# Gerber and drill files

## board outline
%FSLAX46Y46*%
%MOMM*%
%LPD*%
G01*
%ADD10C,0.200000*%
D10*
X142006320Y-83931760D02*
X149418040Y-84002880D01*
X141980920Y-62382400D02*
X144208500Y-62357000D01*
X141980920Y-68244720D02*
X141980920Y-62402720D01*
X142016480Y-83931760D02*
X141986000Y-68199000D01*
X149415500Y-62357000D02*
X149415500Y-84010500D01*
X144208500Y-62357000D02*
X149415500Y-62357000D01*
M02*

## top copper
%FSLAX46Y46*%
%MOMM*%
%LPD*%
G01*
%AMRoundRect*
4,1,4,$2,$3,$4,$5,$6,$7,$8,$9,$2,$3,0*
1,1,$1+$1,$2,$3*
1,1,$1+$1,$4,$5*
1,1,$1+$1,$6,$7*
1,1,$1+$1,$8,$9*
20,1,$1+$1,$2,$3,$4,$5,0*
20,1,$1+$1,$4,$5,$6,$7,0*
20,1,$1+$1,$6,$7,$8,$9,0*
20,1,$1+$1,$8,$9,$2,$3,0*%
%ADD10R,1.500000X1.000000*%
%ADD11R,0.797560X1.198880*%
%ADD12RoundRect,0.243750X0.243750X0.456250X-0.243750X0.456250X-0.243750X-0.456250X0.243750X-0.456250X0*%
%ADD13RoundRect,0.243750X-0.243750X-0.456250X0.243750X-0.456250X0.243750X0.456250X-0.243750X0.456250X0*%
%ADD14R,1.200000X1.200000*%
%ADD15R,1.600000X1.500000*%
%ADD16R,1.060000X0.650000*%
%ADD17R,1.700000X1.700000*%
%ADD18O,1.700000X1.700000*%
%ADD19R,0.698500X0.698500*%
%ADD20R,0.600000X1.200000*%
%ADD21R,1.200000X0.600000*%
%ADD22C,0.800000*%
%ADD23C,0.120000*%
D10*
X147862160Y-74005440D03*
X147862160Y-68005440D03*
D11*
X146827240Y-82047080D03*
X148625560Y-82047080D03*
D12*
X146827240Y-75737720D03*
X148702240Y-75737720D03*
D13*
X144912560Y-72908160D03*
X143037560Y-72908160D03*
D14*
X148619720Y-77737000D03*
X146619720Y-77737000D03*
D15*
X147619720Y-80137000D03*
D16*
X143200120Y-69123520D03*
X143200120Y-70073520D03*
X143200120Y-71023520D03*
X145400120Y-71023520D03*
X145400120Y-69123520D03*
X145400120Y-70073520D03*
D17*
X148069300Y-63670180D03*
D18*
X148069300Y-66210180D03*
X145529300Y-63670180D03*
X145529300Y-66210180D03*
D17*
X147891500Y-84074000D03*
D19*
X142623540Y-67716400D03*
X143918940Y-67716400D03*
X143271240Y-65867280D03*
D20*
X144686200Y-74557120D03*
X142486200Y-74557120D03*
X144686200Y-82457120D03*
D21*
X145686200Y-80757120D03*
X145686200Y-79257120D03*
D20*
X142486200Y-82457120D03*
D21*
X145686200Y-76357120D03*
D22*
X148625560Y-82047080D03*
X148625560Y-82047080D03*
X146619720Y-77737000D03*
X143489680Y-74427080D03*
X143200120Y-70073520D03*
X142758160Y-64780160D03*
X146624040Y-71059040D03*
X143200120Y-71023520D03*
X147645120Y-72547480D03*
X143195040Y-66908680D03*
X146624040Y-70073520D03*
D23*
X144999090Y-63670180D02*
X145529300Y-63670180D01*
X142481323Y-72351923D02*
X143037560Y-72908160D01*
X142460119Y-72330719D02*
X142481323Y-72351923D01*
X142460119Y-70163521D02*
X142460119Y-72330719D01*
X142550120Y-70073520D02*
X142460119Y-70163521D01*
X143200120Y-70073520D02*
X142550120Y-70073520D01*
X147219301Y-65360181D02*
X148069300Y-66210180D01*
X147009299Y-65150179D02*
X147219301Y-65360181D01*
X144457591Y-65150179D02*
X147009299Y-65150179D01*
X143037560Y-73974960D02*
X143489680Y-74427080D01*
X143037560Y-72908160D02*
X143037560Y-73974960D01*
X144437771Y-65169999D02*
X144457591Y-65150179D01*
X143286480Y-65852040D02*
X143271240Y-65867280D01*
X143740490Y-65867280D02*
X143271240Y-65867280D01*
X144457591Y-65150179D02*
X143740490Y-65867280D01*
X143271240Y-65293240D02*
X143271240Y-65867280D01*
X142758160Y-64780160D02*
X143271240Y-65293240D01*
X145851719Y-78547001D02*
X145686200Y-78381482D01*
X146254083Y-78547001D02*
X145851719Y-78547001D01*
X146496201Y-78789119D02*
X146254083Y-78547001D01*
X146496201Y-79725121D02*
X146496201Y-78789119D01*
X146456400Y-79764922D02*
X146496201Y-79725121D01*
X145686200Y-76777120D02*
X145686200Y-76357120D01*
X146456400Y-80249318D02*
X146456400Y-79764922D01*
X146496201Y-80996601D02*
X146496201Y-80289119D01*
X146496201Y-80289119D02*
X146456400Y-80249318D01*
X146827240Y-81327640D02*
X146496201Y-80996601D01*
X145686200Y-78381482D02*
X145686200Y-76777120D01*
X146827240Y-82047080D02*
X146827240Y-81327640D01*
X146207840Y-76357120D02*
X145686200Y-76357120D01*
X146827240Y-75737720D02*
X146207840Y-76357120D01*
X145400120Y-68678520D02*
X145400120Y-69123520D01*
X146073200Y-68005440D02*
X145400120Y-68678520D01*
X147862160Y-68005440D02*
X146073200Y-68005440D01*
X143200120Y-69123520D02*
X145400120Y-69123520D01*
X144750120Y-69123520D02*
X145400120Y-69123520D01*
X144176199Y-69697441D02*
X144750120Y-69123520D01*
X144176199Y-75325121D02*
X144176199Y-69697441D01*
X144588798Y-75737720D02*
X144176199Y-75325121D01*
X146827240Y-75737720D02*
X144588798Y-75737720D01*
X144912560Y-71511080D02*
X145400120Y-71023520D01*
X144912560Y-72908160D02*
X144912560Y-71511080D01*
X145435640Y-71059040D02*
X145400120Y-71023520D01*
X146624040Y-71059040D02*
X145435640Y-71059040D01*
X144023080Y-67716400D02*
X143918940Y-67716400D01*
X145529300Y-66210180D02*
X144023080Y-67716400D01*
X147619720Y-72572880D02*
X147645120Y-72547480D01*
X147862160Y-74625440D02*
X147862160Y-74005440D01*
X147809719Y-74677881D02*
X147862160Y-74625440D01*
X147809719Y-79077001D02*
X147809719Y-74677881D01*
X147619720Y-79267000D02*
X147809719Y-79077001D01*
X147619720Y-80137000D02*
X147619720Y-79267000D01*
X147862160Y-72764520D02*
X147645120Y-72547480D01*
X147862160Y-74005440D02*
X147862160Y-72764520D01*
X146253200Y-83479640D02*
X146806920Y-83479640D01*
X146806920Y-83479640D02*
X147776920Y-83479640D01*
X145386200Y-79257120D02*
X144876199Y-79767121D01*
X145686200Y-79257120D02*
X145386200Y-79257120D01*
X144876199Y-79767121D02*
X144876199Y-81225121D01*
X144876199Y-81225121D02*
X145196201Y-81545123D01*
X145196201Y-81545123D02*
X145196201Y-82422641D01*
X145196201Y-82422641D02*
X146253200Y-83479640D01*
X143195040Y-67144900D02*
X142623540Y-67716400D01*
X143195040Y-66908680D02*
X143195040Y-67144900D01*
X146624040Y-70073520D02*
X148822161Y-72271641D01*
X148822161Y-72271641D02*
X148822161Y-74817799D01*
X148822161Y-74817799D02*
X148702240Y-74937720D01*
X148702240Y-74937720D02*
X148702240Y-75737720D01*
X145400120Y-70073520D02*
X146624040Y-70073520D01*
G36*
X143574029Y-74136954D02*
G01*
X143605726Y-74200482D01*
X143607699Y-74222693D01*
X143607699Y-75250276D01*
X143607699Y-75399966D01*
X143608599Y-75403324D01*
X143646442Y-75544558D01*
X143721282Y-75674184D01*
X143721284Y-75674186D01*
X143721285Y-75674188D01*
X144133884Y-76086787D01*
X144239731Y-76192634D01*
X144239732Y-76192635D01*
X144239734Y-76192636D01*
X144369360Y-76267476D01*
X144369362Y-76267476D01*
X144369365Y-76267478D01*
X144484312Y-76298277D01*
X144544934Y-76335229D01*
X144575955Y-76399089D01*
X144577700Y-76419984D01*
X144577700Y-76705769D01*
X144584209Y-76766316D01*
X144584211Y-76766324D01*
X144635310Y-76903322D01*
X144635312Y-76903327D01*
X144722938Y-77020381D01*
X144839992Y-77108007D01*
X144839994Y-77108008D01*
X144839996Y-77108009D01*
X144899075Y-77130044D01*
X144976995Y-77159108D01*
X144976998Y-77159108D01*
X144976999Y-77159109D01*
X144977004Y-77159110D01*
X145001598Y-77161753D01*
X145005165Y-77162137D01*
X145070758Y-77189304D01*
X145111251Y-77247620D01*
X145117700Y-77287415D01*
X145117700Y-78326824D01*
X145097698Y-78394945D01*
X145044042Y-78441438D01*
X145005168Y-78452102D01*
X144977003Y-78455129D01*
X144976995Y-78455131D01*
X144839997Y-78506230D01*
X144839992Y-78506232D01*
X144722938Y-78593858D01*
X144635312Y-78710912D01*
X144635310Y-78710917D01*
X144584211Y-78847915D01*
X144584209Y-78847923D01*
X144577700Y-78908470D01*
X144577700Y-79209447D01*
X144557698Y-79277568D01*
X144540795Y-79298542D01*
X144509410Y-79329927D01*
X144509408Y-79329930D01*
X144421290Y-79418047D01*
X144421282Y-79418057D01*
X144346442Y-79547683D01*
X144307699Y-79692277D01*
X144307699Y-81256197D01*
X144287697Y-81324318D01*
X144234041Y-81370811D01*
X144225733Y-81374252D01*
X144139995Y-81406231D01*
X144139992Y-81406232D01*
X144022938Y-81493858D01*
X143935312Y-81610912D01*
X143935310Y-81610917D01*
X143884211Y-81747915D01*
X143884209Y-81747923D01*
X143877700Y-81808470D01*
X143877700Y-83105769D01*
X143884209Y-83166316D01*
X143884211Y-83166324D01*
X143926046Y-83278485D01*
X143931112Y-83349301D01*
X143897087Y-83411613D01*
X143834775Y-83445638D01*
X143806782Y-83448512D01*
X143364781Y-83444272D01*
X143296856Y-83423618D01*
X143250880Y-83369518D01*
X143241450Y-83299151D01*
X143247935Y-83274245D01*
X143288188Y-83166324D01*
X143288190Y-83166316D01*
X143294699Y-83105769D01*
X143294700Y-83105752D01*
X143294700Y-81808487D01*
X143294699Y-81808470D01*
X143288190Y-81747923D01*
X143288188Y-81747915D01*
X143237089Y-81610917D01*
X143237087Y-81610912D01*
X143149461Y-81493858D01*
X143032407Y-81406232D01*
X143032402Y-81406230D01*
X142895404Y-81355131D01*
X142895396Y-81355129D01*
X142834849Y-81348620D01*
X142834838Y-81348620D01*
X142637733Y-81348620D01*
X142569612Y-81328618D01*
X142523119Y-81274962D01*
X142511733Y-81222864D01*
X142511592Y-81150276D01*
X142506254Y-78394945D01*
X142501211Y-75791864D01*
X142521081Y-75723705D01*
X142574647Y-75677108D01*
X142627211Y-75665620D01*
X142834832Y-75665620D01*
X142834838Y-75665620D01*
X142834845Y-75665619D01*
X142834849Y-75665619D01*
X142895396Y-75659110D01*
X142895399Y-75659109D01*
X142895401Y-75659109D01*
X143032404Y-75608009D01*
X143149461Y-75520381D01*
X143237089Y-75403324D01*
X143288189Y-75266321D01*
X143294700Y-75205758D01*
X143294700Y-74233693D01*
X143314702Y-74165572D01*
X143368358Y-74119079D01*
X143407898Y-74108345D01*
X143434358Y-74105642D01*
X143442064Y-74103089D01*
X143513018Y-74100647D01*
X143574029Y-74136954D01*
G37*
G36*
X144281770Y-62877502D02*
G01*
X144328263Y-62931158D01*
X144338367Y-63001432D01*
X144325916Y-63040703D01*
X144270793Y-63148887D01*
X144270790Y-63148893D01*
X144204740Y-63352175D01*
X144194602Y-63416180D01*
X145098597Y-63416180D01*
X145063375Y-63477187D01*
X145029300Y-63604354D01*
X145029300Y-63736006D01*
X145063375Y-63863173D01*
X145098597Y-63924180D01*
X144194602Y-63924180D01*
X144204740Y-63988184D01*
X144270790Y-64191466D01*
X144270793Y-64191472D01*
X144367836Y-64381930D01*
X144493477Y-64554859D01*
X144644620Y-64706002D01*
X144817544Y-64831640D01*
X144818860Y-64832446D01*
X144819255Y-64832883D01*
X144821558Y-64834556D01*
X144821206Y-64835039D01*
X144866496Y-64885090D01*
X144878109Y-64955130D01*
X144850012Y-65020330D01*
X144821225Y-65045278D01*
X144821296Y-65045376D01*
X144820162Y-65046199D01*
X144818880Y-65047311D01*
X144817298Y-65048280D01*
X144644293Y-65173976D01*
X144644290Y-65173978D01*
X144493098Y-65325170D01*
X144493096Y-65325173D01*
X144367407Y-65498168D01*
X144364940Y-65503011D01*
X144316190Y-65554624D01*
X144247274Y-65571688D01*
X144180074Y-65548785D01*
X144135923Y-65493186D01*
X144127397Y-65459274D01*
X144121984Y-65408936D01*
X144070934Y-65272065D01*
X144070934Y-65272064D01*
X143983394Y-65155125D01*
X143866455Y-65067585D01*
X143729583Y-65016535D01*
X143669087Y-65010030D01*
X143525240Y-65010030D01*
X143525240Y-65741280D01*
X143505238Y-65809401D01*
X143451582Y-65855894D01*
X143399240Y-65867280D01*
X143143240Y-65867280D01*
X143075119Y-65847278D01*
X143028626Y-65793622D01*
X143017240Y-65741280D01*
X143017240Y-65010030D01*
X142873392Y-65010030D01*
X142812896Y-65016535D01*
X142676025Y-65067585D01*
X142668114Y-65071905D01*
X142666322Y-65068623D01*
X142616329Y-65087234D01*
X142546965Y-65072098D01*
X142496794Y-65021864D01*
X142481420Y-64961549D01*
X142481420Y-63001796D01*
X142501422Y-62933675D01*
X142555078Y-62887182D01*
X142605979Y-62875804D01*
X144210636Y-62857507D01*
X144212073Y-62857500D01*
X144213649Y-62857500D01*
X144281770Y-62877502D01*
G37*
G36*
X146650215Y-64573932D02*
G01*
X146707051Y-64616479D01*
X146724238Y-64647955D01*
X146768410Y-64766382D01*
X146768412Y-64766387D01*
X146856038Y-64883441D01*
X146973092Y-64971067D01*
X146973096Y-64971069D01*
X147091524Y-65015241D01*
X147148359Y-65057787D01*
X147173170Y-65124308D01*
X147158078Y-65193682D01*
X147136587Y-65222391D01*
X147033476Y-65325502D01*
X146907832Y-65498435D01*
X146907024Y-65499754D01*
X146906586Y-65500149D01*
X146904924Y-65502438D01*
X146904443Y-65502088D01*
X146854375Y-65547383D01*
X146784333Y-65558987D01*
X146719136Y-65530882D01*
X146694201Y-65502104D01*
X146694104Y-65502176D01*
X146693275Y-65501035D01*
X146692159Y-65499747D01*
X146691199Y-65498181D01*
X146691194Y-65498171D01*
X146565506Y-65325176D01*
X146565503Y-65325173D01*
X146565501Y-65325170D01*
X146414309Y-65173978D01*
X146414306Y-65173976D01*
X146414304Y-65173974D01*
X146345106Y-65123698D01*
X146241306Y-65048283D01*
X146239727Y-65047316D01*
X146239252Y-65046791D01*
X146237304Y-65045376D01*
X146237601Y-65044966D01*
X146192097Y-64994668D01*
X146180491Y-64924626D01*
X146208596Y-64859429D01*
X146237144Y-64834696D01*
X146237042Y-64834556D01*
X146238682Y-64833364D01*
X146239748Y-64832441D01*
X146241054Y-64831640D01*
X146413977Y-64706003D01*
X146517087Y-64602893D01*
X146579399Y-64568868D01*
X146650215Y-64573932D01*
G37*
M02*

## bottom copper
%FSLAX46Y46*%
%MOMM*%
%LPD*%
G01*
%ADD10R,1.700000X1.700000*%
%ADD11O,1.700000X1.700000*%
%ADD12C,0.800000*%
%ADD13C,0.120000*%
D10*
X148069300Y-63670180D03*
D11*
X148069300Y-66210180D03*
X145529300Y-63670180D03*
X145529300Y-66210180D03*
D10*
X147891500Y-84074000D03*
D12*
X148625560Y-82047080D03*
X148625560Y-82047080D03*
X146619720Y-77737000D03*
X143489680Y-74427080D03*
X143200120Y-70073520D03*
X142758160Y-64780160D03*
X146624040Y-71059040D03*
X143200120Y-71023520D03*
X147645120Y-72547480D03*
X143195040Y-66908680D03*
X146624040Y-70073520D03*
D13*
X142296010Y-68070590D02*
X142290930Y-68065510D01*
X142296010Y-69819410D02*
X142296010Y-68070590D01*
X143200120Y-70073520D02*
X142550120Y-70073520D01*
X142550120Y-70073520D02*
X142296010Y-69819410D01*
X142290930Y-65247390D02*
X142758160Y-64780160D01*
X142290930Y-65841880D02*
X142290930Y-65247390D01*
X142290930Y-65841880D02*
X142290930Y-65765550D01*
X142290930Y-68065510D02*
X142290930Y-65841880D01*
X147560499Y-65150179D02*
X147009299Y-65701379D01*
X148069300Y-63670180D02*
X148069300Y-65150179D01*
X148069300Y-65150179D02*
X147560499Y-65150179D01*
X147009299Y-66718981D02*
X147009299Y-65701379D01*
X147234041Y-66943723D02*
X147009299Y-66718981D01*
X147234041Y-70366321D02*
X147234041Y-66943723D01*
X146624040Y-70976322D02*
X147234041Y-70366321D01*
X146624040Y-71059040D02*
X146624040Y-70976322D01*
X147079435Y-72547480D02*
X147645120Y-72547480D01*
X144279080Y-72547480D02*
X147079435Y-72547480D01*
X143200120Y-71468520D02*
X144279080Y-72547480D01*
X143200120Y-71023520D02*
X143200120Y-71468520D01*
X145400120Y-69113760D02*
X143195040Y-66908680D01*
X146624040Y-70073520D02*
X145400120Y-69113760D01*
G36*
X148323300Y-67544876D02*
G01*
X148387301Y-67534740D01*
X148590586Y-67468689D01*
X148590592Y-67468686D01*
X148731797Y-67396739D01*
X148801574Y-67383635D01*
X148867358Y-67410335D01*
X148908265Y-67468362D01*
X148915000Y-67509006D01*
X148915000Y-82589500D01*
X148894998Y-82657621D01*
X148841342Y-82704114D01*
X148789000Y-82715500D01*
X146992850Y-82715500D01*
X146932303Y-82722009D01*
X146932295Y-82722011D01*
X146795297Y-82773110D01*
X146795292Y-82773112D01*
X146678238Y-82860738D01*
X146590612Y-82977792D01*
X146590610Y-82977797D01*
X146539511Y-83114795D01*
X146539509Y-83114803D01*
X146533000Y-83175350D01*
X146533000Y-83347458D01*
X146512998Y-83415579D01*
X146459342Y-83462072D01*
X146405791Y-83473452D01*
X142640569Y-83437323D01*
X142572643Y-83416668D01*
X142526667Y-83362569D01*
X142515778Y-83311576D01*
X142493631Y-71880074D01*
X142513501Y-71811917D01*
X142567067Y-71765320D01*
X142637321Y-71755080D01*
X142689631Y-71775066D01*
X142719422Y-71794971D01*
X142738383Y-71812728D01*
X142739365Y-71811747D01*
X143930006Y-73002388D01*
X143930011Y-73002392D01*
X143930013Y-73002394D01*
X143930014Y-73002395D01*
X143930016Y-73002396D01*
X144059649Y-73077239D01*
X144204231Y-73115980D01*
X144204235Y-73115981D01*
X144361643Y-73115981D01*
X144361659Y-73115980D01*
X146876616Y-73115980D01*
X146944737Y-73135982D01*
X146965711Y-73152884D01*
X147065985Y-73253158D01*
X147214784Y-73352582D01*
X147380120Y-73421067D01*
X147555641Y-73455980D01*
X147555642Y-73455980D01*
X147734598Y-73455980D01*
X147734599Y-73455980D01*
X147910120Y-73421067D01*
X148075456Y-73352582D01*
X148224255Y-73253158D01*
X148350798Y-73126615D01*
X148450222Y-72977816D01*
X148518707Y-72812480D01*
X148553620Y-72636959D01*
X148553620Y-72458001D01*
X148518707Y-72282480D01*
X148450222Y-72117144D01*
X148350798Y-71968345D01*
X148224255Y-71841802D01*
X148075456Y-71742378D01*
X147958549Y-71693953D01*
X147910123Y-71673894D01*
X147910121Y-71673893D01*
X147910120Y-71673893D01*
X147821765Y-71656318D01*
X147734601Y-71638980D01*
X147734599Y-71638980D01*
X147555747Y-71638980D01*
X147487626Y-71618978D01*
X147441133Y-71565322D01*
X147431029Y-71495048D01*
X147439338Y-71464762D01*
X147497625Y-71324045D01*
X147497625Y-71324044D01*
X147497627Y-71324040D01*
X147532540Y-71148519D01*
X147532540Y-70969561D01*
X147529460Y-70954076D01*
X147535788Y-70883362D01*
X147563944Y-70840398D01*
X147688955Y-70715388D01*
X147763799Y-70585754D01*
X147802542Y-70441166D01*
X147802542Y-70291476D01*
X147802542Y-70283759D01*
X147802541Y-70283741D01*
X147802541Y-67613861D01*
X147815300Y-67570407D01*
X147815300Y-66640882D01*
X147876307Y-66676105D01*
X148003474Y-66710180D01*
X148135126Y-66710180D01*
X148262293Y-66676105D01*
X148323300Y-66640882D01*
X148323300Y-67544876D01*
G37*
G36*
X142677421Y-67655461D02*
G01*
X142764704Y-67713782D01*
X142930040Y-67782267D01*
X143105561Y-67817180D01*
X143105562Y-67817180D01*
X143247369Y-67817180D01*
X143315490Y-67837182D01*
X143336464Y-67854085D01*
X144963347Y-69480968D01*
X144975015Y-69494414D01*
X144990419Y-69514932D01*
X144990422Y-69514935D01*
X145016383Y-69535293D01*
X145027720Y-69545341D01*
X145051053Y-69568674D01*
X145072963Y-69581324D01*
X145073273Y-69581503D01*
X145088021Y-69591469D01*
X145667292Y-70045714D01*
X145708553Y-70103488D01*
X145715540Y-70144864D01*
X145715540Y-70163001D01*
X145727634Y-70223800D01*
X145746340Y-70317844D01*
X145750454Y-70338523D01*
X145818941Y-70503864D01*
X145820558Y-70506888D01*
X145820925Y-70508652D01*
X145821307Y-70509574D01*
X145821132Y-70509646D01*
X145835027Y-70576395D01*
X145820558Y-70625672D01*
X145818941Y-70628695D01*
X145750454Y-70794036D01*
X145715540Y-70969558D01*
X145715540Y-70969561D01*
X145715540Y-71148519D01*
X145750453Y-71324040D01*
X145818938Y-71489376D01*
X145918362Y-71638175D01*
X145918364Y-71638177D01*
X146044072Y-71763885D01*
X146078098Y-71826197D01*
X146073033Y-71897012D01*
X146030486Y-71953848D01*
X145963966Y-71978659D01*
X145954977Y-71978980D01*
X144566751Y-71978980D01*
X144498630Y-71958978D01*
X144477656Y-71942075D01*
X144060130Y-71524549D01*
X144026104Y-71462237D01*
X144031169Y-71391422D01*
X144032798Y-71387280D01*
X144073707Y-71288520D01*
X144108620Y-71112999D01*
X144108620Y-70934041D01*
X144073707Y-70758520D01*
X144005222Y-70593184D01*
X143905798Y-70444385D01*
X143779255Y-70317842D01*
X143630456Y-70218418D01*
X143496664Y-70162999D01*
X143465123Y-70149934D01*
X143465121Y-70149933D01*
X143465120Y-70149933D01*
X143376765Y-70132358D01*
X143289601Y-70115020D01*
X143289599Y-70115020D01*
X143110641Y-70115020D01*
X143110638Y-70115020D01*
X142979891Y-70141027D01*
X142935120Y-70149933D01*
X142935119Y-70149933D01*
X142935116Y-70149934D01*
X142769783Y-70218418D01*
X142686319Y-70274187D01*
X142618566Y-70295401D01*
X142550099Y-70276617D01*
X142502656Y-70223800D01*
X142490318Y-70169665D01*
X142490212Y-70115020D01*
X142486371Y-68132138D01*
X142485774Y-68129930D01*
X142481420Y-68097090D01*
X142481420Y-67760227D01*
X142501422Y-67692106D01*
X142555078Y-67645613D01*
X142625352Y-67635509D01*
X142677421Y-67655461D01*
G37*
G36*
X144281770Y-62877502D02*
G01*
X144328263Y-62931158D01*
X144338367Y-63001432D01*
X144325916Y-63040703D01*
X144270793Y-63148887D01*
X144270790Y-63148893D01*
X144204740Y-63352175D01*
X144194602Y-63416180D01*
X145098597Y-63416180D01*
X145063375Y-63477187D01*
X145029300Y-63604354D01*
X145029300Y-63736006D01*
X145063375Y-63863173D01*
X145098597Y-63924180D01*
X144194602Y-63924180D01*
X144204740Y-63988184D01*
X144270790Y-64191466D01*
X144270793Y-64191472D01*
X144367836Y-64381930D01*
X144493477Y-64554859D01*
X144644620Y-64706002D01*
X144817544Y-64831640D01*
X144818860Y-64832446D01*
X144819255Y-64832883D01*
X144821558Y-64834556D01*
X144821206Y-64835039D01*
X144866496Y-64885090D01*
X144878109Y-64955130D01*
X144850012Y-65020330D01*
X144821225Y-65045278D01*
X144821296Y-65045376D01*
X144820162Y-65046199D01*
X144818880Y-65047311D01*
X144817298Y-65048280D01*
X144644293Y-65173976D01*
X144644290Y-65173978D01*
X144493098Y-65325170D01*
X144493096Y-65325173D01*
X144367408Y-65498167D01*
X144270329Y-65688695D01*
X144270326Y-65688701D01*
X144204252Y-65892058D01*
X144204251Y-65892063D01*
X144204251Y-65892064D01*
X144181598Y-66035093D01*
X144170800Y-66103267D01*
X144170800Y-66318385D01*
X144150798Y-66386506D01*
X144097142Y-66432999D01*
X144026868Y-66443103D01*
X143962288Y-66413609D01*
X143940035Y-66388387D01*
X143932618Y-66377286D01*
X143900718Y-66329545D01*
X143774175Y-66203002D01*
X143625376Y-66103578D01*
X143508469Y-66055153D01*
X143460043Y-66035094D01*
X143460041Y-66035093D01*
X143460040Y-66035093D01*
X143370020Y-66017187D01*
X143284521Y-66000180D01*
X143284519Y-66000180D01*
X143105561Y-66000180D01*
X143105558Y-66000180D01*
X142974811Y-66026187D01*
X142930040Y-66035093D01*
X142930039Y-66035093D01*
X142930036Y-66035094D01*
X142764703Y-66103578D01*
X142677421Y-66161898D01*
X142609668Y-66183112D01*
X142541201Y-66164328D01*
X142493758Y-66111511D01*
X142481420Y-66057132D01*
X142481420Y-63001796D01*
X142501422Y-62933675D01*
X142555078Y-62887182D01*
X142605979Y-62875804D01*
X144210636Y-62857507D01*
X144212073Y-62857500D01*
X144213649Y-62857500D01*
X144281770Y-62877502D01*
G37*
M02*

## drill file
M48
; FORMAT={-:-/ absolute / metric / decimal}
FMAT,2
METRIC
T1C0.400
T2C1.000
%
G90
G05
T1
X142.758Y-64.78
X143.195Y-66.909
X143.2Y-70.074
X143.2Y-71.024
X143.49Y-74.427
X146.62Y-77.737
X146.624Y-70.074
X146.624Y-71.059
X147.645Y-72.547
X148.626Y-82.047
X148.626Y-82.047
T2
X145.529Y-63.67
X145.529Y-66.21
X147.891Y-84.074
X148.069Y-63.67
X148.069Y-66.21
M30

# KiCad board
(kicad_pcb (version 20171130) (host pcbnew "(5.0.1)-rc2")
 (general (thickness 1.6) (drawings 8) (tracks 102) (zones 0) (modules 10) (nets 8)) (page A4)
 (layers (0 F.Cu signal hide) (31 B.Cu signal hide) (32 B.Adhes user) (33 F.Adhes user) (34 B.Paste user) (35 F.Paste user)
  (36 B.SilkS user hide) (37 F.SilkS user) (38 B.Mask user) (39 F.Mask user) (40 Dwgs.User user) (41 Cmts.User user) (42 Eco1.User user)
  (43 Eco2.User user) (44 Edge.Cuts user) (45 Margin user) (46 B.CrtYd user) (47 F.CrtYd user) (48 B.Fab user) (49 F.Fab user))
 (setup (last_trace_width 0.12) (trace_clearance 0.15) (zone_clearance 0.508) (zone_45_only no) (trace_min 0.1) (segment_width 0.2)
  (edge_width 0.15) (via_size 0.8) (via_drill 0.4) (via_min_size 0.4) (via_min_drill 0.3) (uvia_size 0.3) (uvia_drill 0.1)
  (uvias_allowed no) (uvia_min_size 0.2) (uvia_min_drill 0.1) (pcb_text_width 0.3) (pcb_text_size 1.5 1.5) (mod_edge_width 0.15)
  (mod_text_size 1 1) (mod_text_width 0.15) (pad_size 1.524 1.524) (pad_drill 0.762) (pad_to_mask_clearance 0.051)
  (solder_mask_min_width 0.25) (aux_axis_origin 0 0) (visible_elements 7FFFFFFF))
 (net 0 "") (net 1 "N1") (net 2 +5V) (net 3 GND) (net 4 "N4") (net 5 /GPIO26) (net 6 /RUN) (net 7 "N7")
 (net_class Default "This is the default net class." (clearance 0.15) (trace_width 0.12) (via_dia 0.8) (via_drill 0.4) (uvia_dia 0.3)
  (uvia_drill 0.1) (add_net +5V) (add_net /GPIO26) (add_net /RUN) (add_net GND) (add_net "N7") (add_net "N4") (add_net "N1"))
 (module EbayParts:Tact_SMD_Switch (layer F.Cu) (at 149.36216 74.00544 90)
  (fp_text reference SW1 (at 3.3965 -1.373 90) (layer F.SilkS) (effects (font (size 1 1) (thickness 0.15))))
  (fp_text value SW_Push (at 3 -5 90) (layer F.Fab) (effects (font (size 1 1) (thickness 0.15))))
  (pad 1 smd rect (at 0 -1.5 90) (size 1 1.5) (layers F.Cu F.Paste F.Mask) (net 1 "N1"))
  (pad 2 smd rect (at 6 -1.5 90) (size 1 1.5) (layers F.Cu F.Paste F.Mask) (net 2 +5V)))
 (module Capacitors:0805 (layer F.Cu) (at 147.7264 82.04708 180)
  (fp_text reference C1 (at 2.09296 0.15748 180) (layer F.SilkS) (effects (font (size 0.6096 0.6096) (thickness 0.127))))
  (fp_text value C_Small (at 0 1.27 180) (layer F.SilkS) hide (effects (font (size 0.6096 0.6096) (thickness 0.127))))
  (pad 2 smd rect (at 0.89916 0 180) (size 0.79756 1.19888) (layers F.Cu F.Paste F.Mask) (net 2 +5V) (solder_mask_margin 0.1016))
  (pad 1 smd rect (at -0.89916 0 180) (size 0.79756 1.19888) (layers F.Cu F.Paste F.Mask) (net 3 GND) (solder_mask_margin 0.1016)))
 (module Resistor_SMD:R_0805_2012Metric (layer F.Cu) (at 147.76474 75.73772 180)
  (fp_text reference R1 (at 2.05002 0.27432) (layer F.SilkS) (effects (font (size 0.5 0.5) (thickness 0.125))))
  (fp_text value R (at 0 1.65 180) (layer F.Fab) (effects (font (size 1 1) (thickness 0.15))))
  (pad 2 smd roundrect (at 0.9375 0 180) (size 0.975 1.4) (layers F.Cu F.Paste F.Mask) (roundrect_rratio 0.25) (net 2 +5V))
  (pad 1 smd roundrect (at -0.9375 0 180) (size 0.975 1.4) (layers F.Cu F.Paste F.Mask) (roundrect_rratio 0.25) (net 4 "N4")))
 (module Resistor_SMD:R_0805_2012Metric (layer F.Cu) (at 143.97506 72.90816)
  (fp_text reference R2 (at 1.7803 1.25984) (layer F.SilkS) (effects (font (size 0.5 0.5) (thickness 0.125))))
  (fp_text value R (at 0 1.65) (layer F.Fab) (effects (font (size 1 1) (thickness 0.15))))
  (pad 2 smd roundrect (at 0.9375 0) (size 0.975 1.4) (layers F.Cu F.Paste F.Mask) (roundrect_rratio 0.25) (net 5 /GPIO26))
  (pad 1 smd roundrect (at -0.9375 0) (size 0.975 1.4) (layers F.Cu F.Paste F.Mask) (roundrect_rratio 0.25) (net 3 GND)))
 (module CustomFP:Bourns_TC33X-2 (layer F.Cu) (at 147.61972 80.137 180)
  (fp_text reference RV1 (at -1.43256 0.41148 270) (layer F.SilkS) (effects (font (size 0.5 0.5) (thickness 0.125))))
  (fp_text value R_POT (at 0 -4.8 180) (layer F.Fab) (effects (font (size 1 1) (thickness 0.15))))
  (pad 3 smd rect (at -1 2.4 180) (size 1.2 1.2) (layers F.Cu F.Paste F.Mask))
  (pad 2 smd rect (at 1 2.4 180) (size 1.2 1.2) (layers F.Cu F.Paste F.Mask) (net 3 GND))
  (pad 1 smd rect (at 0 0 180) (size 1.6 1.5) (layers F.Cu F.Paste F.Mask) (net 1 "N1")))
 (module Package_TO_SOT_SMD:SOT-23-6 (layer F.Cu) (at 144.30012 70.07352)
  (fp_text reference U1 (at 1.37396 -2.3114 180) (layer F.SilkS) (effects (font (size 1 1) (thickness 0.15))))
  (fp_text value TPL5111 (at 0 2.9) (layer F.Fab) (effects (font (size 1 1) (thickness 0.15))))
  (pad 1 smd rect (at -1.1 -0.95) (size 1.06 0.65) (layers F.Cu F.Paste F.Mask) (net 2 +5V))
  (pad 2 smd rect (at -1.1 0) (size 1.06 0.65) (layers F.Cu F.Paste F.Mask) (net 3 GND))
  (pad 3 smd rect (at -1.1 0.95) (size 1.06 0.65) (layers F.Cu F.Paste F.Mask) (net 1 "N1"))
  (pad 4 smd rect (at 1.1 0.95) (size 1.06 0.65) (layers F.Cu F.Paste F.Mask) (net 5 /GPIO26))
  (pad 6 smd rect (at 1.1 -0.95) (size 1.06 0.65) (layers F.Cu F.Paste F.Mask) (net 2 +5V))
  (pad 5 smd rect (at 1.1 0) (size 1.06 0.65) (layers F.Cu F.Paste F.Mask) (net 4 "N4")))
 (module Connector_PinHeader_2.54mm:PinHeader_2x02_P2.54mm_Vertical (layer F.Cu) (at 148.0693 63.67018 270)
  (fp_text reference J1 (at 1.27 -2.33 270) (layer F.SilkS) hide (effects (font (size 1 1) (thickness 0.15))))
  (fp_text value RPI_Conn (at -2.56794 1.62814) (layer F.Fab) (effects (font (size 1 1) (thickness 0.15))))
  (pad 1 thru_hole rect (at 0 0 270) (size 1.7 1.7) (drill 1) (layers *.Cu *.Mask) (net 5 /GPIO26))
  (pad 2 thru_hole oval (at 2.54 0 270) (size 1.7 1.7) (drill 1) (layers *.Cu *.Mask) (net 3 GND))
  (pad 3 thru_hole oval (at 0 2.54 270) (size 1.7 1.7) (drill 1) (layers *.Cu *.Mask) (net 3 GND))
  (pad 4 thru_hole oval (at 2.54 2.54 270) (size 1.7 1.7) (drill 1) (layers *.Cu *.Mask) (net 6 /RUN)))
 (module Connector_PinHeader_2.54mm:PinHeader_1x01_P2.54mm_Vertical (layer F.Cu) (at 147.8915 84.074)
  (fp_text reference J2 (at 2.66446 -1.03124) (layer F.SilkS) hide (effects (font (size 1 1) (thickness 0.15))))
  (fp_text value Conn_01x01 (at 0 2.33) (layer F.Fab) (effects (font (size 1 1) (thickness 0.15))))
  (pad 1 thru_hole rect (at 0 0) (size 1.7 1.7) (drill 1) (layers *.Cu *.Mask) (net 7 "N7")))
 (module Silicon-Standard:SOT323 (layer F.Cu) (at 143.27124 66.79184)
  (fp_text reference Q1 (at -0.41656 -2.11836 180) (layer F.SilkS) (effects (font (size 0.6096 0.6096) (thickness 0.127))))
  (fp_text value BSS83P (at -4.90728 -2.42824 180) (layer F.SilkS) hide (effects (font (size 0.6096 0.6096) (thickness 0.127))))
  (pad 1 smd rect (at -0.6477 0.92456) (size 0.6985 0.6985) (layers F.Cu F.Paste F.Mask) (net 4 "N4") (solder_mask_margin 0.1016))
  (pad 2 smd rect (at 0.6477 0.92456) (size 0.6985 0.6985) (layers F.Cu F.Paste F.Mask) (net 6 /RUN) (solder_mask_margin 0.1016))
  (pad 3 smd rect (at 0 -0.92456) (size 0.6985 0.6985) (layers F.Cu F.Paste F.Mask) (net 3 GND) (solder_mask_margin 0.1016)))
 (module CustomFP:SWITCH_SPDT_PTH (layer F.Cu) (at 143.5862 78.55712)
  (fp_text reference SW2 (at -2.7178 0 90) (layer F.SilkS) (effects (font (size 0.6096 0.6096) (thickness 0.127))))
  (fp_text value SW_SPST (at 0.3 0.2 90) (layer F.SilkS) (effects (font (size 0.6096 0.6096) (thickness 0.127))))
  (pad "" smd rect (at 1.1 -4 90) (size 1.2 0.6) (layers F.Cu F.Paste F.Mask) (solder_mask_margin 0.1016))
  (pad "" smd rect (at -1.1 -4 90) (size 1.2 0.6) (layers F.Cu F.Paste F.Mask) (solder_mask_margin 0.1016))
  (pad "" smd rect (at 1.1 3.9 90) (size 1.2 0.6) (layers F.Cu F.Paste F.Mask) (solder_mask_margin 0.1016))
  (pad 3 smd rect (at 2.1 2.2) (size 1.2 0.6) (layers F.Cu F.Paste F.Mask) (solder_mask_margin 0.1016))
  (pad 2 smd rect (at 2.1 0.7) (size 1.2 0.6) (layers F.Cu F.Paste F.Mask) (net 7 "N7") (solder_mask_margin 0.1016))
  (pad "" smd rect (at -1.1 3.9 90) (size 1.2 0.6) (layers F.Cu F.Paste F.Mask) (solder_mask_margin 0.1016))
  (pad 1 smd rect (at 2.1 -2.2) (size 1.2 0.6) (layers F.Cu F.Paste F.Mask) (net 2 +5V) (solder_mask_margin 0.1016)))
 (gr_line (start 142.00632 83.93176) (end 149.41804 84.00288) (layer Edge.Cuts) (width 0.2))
 (gr_line (start 141.98092 62.3824) (end 144.2085 62.357) (layer Edge.Cuts) (width 0.2))
 (gr_line (start 141.98092 68.24472) (end 141.98092 62.40272) (layer Edge.Cuts) (width 0.2))
 (gr_line (start 142.01648 83.93176) (end 141.986 68.199) (layer Edge.Cuts) (width 0.2))
 (gr_line (start 149.4155 62.357) (end 149.4155 84.0105) (layer Edge.Cuts) (width 0.2))
 (gr_line (start 144.2085 62.357) (end 149.4155 62.357) (layer Edge.Cuts) (width 0.2))
 (segment (start 144.99909 63.67018) (end 145.5293 63.67018) (width 0.12) (layer F.Cu) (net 3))
 (via (at 148.62556 82.04708) (size 0.8) (drill 0.4) (layers F.Cu B.Cu) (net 3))
 (via (at 148.62556 82.04708) (size 0.8) (drill 0.4) (layers F.Cu B.Cu) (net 3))
 (via (at 146.61972 77.737) (size 0.8) (drill 0.4) (layers F.Cu B.Cu) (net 3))
 (via (at 143.48968 74.42708) (size 0.8) (drill 0.4) (layers F.Cu B.Cu) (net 3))
 (segment (start 142.481323 72.351923) (end 143.03756 72.90816) (width 0.12) (layer F.Cu) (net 3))
 (segment (start 142.460119 72.330719) (end 142.481323 72.351923) (width 0.12) (layer F.Cu) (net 3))
 (segment (start 142.460119 70.163521) (end 142.460119 72.330719) (width 0.12) (layer F.Cu) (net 3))
 (segment (start 142.55012 70.07352) (end 142.460119 70.163521) (width 0.12) (layer F.Cu) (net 3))
 (segment (start 143.20012 70.07352) (end 142.55012 70.07352) (width 0.12) (layer F.Cu) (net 3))
 (via (at 143.20012 70.07352) (size 0.8) (drill 0.4) (layers F.Cu B.Cu) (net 3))
 (segment (start 147.219301 65.360181) (end 148.0693 66.21018) (width 0.12) (layer F.Cu) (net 3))
 (segment (start 147.009299 65.150179) (end 147.219301 65.360181) (width 0.12) (layer F.Cu) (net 3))
 (segment (start 144.457591 65.150179) (end 147.009299 65.150179) (width 0.12) (layer F.Cu) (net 3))
 (segment (start 143.03756 73.97496) (end 143.48968 74.42708) (width 0.12) (layer F.Cu) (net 3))
 (segment (start 143.03756 72.90816) (end 143.03756 73.97496) (width 0.12) (layer F.Cu) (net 3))
 (segment (start 142.29601 68.07059) (end 142.29093 68.06551) (width 0.12) (layer B.Cu) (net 3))
 (segment (start 142.29601 69.81941) (end 142.29601 68.07059) (width 0.12) (layer B.Cu) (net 3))
 (segment (start 143.20012 70.07352) (end 142.55012 70.07352) (width 0.12) (layer B.Cu) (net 3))
 (segment (start 142.55012 70.07352) (end 142.29601 69.81941) (width 0.12) (layer B.Cu) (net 3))
 (segment (start 144.437771 65.169999) (end 144.457591 65.150179) (width 0.12) (layer F.Cu) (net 3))
 (segment (start 143.28648 65.85204) (end 143.27124 65.86728) (width 0.12) (layer F.Cu) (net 3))
 (segment (start 143.74049 65.86728) (end 143.27124 65.86728) (width 0.12) (layer F.Cu) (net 3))
 (segment (start 144.457591 65.150179) (end 143.74049 65.86728) (width 0.12) (layer F.Cu) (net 3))
 (via (at 142.75816 64.78016) (size 0.8) (drill 0.4) (layers F.Cu B.Cu) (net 3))
 (segment (start 142.29093 65.24739) (end 142.75816 64.78016) (width 0.12) (layer B.Cu) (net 3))
 (segment (start 142.29093 65.84188) (end 142.29093 65.24739) (width 0.12) (layer B.Cu) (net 3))
 (segment (start 142.29093 65.84188) (end 142.29093 65.76555) (width 0.12) (layer B.Cu) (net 3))
 (segment (start 142.29093 68.06551) (end 142.29093 65.84188) (width 0.12) (layer B.Cu) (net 3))
 (segment (start 143.27124 65.29324) (end 143.27124 65.86728) (width 0.12) (layer F.Cu) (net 3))
 (segment (start 142.75816 64.78016) (end 143.27124 65.29324) (width 0.12) (layer F.Cu) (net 3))
 (segment (start 145.851719 78.547001) (end 145.6862 78.381482) (width 0.12) (layer F.Cu) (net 2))
 (segment (start 146.254083 78.547001) (end 145.851719 78.547001) (width 0.12) (layer F.Cu) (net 2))
 (segment (start 146.496201 78.789119) (end 146.254083 78.547001) (width 0.12) (layer F.Cu) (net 2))
 (segment (start 146.496201 79.725121) (end 146.496201 78.789119) (width 0.12) (layer F.Cu) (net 2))
 (segment (start 146.4564 79.764922) (end 146.496201 79.725121) (width 0.12) (layer F.Cu) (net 2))
 (segment (start 145.6862 76.77712) (end 145.6862 76.35712) (width 0.12) (layer F.Cu) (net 2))
 (segment (start 146.4564 80.249318) (end 146.4564 79.764922) (width 0.12) (layer F.Cu) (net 2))
 (segment (start 146.496201 80.996601) (end 146.496201 80.289119) (width 0.12) (layer F.Cu) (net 2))
 (segment (start 146.496201 80.289119) (end 146.4564 80.249318) (width 0.12) (layer F.Cu) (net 2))
 (segment (start 146.82724 81.32764) (end 146.496201 80.996601) (width 0.12) (layer F.Cu) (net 2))
 (segment (start 145.6862 78.381482) (end 145.6862 76.77712) (width 0.12) (layer F.Cu) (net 2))
 (segment (start 146.82724 82.04708) (end 146.82724 81.32764) (width 0.12) (layer F.Cu) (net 2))
 (segment (start 146.20784 76.35712) (end 145.6862 76.35712) (width 0.12) (layer F.Cu) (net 2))
 (segment (start 146.82724 75.73772) (end 146.20784 76.35712) (width 0.12) (layer F.Cu) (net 2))
 (segment (start 145.40012 68.67852) (end 145.40012 69.12352) (width 0.12) (layer F.Cu) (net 2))
 (segment (start 146.0732 68.00544) (end 145.40012 68.67852) (width 0.12) (layer F.Cu) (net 2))
 (segment (start 147.86216 68.00544) (end 146.0732 68.00544) (width 0.12) (layer F.Cu) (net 2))
 (segment (start 143.20012 69.12352) (end 145.40012 69.12352) (width 0.12) (layer F.Cu) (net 2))
 (segment (start 144.75012 69.12352) (end 145.40012 69.12352) (width 0.12) (layer F.Cu) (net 2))
 (segment (start 144.176199 69.697441) (end 144.75012 69.12352) (width 0.12) (layer F.Cu) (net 2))
 (segment (start 144.176199 75.325121) (end 144.176199 69.697441) (width 0.12) (layer F.Cu) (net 2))
 (segment (start 144.588798 75.73772) (end 144.176199 75.325121) (width 0.12) (layer F.Cu) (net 2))
 (segment (start 146.82724 75.73772) (end 144.588798 75.73772) (width 0.12) (layer F.Cu) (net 2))
 (segment (start 144.91256 71.51108) (end 145.40012 71.02352) (width 0.12) (layer F.Cu) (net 5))
 (segment (start 144.91256 72.90816) (end 144.91256 71.51108) (width 0.12) (layer F.Cu) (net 5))
 (via (at 146.62404 71.05904) (size 0.8) (drill 0.4) (layers F.Cu B.Cu) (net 5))
 (segment (start 147.560499 65.150179) (end 147.009299 65.701379) (width 0.12) (layer B.Cu) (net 5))
 (segment (start 148.0693 63.67018) (end 148.0693 65.150179) (width 0.12) (layer B.Cu) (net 5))
 (segment (start 148.0693 65.150179) (end 147.560499 65.150179) (width 0.12) (layer B.Cu) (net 5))
 (segment (start 145.43564 71.05904) (end 145.40012 71.02352) (width 0.12) (layer F.Cu) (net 5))
 (segment (start 146.62404 71.05904) (end 145.43564 71.05904) (width 0.12) (layer F.Cu) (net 5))
 (segment (start 147.009299 66.718981) (end 147.009299 65.701379) (width 0.12) (layer B.Cu) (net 5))
 (segment (start 147.234041 66.943723) (end 147.009299 66.718981) (width 0.12) (layer B.Cu) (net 5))
 (segment (start 147.234041 70.366321) (end 147.234041 66.943723) (width 0.12) (layer B.Cu) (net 5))
 (segment (start 146.62404 70.976322) (end 147.234041 70.366321) (width 0.12) (layer B.Cu) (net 5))
 (segment (start 146.62404 71.05904) (end 146.62404 70.976322) (width 0.12) (layer B.Cu) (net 5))
 (segment (start 144.02308 67.7164) (end 143.91894 67.7164) (width 0.12) (layer F.Cu) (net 6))
 (segment (start 145.5293 66.21018) (end 144.02308 67.7164) (width 0.12) (layer F.Cu) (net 6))
 (via (at 143.20012 71.02352) (size 0.8) (drill 0.4) (layers F.Cu B.Cu) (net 1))
 (via (at 147.64512 72.54748) (size 0.8) (drill 0.4) (layers F.Cu B.Cu) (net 1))
 (segment (start 147.61972 72.57288) (end 147.64512 72.54748) (width 0.12) (layer F.Cu) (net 1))
 (segment (start 147.079435 72.54748) (end 147.64512 72.54748) (width 0.12) (layer B.Cu) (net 1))
 (segment (start 144.27908 72.54748) (end 147.079435 72.54748) (width 0.12) (layer B.Cu) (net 1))
 (segment (start 143.20012 71.46852) (end 144.27908 72.54748) (width 0.12) (layer B.Cu) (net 1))
 (segment (start 143.20012 71.02352) (end 143.20012 71.46852) (width 0.12) (layer B.Cu) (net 1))
 (segment (start 147.86216 74.62544) (end 147.86216 74.00544) (width 0.12) (layer F.Cu) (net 1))
 (segment (start 147.809719 74.677881) (end 147.86216 74.62544) (width 0.12) (layer F.Cu) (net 1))
 (segment (start 147.809719 79.077001) (end 147.809719 74.677881) (width 0.12) (layer F.Cu) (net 1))
 (segment (start 147.61972 79.267) (end 147.809719 79.077001) (width 0.12) (layer F.Cu) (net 1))
 (segment (start 147.61972 80.137) (end 147.61972 79.267) (width 0.12) (layer F.Cu) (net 1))
 (segment (start 147.86216 72.76452) (end 147.64512 72.54748) (width 0.12) (layer F.Cu) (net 1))
 (segment (start 147.86216 74.00544) (end 147.86216 72.76452) (width 0.12) (layer F.Cu) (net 1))
 (segment (start 146.2532 83.47964) (end 146.80692 83.47964) (width 0.12) (layer F.Cu) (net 7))
 (segment (start 146.80692 83.47964) (end 147.77692 83.47964) (width 0.12) (layer F.Cu) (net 7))
 (segment (start 145.3862 79.25712) (end 144.876199 79.767121) (width 0.12) (layer F.Cu) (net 7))
 (segment (start 145.6862 79.25712) (end 145.3862 79.25712) (width 0.12) (layer F.Cu) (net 7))
 (segment (start 144.876199 79.767121) (end 144.876199 81.225121) (width 0.12) (layer F.Cu) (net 7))
 (segment (start 144.876199 81.225121) (end 145.196201 81.545123) (width 0.12) (layer F.Cu) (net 7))
 (segment (start 145.196201 81.545123) (end 145.196201 82.422641) (width 0.12) (layer F.Cu) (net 7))
 (segment (start 145.196201 82.422641) (end 146.2532 83.47964) (width 0.12) (layer F.Cu) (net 7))
 (via (at 143.19504 66.90868) (size 0.8) (drill 0.4) (layers F.Cu B.Cu) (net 4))
 (segment (start 143.19504 67.1449) (end 142.62354 67.7164) (width 0.12) (layer F.Cu) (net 4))
 (segment (start 143.19504 66.90868) (end 143.19504 67.1449) (width 0.12) (layer F.Cu) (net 4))
 (segment (start 145.40012 69.11376) (end 143.19504 66.90868) (width 0.12) (layer B.Cu) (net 4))
 (segment (start 146.62404 70.07352) (end 148.822161 72.271641) (width 0.12) (layer F.Cu) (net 4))
 (segment (start 148.822161 72.271641) (end 148.822161 74.817799) (width 0.12) (layer F.Cu) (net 4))
 (segment (start 148.822161 74.817799) (end 148.70224 74.93772) (width 0.12) (layer F.Cu) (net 4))
 (segment (start 148.70224 74.93772) (end 148.70224 75.73772) (width 0.12) (layer F.Cu) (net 4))
 (segment (start 146.62404 70.07352) (end 145.40012 69.11376) (width 0.12) (layer B.Cu) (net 4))
 (via (at 146.62404 70.07352) (size 0.8) (drill 0.4) (layers F.Cu B.Cu) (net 4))
 (segment (start 145.40012 70.07352) (end 146.62404 70.07352) (width 0.12) (layer F.Cu) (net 4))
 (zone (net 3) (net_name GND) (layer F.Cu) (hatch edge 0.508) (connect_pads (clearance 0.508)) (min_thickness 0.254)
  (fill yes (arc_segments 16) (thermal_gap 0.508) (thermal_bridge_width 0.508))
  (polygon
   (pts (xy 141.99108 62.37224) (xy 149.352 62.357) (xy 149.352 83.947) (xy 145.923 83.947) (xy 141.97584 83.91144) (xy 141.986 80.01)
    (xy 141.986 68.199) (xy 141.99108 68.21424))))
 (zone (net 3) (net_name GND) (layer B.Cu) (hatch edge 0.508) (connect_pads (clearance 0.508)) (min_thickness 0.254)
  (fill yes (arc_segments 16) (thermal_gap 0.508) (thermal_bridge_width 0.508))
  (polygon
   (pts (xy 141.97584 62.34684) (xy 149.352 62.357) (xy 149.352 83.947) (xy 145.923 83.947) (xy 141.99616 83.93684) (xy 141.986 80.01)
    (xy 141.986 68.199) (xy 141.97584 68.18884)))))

